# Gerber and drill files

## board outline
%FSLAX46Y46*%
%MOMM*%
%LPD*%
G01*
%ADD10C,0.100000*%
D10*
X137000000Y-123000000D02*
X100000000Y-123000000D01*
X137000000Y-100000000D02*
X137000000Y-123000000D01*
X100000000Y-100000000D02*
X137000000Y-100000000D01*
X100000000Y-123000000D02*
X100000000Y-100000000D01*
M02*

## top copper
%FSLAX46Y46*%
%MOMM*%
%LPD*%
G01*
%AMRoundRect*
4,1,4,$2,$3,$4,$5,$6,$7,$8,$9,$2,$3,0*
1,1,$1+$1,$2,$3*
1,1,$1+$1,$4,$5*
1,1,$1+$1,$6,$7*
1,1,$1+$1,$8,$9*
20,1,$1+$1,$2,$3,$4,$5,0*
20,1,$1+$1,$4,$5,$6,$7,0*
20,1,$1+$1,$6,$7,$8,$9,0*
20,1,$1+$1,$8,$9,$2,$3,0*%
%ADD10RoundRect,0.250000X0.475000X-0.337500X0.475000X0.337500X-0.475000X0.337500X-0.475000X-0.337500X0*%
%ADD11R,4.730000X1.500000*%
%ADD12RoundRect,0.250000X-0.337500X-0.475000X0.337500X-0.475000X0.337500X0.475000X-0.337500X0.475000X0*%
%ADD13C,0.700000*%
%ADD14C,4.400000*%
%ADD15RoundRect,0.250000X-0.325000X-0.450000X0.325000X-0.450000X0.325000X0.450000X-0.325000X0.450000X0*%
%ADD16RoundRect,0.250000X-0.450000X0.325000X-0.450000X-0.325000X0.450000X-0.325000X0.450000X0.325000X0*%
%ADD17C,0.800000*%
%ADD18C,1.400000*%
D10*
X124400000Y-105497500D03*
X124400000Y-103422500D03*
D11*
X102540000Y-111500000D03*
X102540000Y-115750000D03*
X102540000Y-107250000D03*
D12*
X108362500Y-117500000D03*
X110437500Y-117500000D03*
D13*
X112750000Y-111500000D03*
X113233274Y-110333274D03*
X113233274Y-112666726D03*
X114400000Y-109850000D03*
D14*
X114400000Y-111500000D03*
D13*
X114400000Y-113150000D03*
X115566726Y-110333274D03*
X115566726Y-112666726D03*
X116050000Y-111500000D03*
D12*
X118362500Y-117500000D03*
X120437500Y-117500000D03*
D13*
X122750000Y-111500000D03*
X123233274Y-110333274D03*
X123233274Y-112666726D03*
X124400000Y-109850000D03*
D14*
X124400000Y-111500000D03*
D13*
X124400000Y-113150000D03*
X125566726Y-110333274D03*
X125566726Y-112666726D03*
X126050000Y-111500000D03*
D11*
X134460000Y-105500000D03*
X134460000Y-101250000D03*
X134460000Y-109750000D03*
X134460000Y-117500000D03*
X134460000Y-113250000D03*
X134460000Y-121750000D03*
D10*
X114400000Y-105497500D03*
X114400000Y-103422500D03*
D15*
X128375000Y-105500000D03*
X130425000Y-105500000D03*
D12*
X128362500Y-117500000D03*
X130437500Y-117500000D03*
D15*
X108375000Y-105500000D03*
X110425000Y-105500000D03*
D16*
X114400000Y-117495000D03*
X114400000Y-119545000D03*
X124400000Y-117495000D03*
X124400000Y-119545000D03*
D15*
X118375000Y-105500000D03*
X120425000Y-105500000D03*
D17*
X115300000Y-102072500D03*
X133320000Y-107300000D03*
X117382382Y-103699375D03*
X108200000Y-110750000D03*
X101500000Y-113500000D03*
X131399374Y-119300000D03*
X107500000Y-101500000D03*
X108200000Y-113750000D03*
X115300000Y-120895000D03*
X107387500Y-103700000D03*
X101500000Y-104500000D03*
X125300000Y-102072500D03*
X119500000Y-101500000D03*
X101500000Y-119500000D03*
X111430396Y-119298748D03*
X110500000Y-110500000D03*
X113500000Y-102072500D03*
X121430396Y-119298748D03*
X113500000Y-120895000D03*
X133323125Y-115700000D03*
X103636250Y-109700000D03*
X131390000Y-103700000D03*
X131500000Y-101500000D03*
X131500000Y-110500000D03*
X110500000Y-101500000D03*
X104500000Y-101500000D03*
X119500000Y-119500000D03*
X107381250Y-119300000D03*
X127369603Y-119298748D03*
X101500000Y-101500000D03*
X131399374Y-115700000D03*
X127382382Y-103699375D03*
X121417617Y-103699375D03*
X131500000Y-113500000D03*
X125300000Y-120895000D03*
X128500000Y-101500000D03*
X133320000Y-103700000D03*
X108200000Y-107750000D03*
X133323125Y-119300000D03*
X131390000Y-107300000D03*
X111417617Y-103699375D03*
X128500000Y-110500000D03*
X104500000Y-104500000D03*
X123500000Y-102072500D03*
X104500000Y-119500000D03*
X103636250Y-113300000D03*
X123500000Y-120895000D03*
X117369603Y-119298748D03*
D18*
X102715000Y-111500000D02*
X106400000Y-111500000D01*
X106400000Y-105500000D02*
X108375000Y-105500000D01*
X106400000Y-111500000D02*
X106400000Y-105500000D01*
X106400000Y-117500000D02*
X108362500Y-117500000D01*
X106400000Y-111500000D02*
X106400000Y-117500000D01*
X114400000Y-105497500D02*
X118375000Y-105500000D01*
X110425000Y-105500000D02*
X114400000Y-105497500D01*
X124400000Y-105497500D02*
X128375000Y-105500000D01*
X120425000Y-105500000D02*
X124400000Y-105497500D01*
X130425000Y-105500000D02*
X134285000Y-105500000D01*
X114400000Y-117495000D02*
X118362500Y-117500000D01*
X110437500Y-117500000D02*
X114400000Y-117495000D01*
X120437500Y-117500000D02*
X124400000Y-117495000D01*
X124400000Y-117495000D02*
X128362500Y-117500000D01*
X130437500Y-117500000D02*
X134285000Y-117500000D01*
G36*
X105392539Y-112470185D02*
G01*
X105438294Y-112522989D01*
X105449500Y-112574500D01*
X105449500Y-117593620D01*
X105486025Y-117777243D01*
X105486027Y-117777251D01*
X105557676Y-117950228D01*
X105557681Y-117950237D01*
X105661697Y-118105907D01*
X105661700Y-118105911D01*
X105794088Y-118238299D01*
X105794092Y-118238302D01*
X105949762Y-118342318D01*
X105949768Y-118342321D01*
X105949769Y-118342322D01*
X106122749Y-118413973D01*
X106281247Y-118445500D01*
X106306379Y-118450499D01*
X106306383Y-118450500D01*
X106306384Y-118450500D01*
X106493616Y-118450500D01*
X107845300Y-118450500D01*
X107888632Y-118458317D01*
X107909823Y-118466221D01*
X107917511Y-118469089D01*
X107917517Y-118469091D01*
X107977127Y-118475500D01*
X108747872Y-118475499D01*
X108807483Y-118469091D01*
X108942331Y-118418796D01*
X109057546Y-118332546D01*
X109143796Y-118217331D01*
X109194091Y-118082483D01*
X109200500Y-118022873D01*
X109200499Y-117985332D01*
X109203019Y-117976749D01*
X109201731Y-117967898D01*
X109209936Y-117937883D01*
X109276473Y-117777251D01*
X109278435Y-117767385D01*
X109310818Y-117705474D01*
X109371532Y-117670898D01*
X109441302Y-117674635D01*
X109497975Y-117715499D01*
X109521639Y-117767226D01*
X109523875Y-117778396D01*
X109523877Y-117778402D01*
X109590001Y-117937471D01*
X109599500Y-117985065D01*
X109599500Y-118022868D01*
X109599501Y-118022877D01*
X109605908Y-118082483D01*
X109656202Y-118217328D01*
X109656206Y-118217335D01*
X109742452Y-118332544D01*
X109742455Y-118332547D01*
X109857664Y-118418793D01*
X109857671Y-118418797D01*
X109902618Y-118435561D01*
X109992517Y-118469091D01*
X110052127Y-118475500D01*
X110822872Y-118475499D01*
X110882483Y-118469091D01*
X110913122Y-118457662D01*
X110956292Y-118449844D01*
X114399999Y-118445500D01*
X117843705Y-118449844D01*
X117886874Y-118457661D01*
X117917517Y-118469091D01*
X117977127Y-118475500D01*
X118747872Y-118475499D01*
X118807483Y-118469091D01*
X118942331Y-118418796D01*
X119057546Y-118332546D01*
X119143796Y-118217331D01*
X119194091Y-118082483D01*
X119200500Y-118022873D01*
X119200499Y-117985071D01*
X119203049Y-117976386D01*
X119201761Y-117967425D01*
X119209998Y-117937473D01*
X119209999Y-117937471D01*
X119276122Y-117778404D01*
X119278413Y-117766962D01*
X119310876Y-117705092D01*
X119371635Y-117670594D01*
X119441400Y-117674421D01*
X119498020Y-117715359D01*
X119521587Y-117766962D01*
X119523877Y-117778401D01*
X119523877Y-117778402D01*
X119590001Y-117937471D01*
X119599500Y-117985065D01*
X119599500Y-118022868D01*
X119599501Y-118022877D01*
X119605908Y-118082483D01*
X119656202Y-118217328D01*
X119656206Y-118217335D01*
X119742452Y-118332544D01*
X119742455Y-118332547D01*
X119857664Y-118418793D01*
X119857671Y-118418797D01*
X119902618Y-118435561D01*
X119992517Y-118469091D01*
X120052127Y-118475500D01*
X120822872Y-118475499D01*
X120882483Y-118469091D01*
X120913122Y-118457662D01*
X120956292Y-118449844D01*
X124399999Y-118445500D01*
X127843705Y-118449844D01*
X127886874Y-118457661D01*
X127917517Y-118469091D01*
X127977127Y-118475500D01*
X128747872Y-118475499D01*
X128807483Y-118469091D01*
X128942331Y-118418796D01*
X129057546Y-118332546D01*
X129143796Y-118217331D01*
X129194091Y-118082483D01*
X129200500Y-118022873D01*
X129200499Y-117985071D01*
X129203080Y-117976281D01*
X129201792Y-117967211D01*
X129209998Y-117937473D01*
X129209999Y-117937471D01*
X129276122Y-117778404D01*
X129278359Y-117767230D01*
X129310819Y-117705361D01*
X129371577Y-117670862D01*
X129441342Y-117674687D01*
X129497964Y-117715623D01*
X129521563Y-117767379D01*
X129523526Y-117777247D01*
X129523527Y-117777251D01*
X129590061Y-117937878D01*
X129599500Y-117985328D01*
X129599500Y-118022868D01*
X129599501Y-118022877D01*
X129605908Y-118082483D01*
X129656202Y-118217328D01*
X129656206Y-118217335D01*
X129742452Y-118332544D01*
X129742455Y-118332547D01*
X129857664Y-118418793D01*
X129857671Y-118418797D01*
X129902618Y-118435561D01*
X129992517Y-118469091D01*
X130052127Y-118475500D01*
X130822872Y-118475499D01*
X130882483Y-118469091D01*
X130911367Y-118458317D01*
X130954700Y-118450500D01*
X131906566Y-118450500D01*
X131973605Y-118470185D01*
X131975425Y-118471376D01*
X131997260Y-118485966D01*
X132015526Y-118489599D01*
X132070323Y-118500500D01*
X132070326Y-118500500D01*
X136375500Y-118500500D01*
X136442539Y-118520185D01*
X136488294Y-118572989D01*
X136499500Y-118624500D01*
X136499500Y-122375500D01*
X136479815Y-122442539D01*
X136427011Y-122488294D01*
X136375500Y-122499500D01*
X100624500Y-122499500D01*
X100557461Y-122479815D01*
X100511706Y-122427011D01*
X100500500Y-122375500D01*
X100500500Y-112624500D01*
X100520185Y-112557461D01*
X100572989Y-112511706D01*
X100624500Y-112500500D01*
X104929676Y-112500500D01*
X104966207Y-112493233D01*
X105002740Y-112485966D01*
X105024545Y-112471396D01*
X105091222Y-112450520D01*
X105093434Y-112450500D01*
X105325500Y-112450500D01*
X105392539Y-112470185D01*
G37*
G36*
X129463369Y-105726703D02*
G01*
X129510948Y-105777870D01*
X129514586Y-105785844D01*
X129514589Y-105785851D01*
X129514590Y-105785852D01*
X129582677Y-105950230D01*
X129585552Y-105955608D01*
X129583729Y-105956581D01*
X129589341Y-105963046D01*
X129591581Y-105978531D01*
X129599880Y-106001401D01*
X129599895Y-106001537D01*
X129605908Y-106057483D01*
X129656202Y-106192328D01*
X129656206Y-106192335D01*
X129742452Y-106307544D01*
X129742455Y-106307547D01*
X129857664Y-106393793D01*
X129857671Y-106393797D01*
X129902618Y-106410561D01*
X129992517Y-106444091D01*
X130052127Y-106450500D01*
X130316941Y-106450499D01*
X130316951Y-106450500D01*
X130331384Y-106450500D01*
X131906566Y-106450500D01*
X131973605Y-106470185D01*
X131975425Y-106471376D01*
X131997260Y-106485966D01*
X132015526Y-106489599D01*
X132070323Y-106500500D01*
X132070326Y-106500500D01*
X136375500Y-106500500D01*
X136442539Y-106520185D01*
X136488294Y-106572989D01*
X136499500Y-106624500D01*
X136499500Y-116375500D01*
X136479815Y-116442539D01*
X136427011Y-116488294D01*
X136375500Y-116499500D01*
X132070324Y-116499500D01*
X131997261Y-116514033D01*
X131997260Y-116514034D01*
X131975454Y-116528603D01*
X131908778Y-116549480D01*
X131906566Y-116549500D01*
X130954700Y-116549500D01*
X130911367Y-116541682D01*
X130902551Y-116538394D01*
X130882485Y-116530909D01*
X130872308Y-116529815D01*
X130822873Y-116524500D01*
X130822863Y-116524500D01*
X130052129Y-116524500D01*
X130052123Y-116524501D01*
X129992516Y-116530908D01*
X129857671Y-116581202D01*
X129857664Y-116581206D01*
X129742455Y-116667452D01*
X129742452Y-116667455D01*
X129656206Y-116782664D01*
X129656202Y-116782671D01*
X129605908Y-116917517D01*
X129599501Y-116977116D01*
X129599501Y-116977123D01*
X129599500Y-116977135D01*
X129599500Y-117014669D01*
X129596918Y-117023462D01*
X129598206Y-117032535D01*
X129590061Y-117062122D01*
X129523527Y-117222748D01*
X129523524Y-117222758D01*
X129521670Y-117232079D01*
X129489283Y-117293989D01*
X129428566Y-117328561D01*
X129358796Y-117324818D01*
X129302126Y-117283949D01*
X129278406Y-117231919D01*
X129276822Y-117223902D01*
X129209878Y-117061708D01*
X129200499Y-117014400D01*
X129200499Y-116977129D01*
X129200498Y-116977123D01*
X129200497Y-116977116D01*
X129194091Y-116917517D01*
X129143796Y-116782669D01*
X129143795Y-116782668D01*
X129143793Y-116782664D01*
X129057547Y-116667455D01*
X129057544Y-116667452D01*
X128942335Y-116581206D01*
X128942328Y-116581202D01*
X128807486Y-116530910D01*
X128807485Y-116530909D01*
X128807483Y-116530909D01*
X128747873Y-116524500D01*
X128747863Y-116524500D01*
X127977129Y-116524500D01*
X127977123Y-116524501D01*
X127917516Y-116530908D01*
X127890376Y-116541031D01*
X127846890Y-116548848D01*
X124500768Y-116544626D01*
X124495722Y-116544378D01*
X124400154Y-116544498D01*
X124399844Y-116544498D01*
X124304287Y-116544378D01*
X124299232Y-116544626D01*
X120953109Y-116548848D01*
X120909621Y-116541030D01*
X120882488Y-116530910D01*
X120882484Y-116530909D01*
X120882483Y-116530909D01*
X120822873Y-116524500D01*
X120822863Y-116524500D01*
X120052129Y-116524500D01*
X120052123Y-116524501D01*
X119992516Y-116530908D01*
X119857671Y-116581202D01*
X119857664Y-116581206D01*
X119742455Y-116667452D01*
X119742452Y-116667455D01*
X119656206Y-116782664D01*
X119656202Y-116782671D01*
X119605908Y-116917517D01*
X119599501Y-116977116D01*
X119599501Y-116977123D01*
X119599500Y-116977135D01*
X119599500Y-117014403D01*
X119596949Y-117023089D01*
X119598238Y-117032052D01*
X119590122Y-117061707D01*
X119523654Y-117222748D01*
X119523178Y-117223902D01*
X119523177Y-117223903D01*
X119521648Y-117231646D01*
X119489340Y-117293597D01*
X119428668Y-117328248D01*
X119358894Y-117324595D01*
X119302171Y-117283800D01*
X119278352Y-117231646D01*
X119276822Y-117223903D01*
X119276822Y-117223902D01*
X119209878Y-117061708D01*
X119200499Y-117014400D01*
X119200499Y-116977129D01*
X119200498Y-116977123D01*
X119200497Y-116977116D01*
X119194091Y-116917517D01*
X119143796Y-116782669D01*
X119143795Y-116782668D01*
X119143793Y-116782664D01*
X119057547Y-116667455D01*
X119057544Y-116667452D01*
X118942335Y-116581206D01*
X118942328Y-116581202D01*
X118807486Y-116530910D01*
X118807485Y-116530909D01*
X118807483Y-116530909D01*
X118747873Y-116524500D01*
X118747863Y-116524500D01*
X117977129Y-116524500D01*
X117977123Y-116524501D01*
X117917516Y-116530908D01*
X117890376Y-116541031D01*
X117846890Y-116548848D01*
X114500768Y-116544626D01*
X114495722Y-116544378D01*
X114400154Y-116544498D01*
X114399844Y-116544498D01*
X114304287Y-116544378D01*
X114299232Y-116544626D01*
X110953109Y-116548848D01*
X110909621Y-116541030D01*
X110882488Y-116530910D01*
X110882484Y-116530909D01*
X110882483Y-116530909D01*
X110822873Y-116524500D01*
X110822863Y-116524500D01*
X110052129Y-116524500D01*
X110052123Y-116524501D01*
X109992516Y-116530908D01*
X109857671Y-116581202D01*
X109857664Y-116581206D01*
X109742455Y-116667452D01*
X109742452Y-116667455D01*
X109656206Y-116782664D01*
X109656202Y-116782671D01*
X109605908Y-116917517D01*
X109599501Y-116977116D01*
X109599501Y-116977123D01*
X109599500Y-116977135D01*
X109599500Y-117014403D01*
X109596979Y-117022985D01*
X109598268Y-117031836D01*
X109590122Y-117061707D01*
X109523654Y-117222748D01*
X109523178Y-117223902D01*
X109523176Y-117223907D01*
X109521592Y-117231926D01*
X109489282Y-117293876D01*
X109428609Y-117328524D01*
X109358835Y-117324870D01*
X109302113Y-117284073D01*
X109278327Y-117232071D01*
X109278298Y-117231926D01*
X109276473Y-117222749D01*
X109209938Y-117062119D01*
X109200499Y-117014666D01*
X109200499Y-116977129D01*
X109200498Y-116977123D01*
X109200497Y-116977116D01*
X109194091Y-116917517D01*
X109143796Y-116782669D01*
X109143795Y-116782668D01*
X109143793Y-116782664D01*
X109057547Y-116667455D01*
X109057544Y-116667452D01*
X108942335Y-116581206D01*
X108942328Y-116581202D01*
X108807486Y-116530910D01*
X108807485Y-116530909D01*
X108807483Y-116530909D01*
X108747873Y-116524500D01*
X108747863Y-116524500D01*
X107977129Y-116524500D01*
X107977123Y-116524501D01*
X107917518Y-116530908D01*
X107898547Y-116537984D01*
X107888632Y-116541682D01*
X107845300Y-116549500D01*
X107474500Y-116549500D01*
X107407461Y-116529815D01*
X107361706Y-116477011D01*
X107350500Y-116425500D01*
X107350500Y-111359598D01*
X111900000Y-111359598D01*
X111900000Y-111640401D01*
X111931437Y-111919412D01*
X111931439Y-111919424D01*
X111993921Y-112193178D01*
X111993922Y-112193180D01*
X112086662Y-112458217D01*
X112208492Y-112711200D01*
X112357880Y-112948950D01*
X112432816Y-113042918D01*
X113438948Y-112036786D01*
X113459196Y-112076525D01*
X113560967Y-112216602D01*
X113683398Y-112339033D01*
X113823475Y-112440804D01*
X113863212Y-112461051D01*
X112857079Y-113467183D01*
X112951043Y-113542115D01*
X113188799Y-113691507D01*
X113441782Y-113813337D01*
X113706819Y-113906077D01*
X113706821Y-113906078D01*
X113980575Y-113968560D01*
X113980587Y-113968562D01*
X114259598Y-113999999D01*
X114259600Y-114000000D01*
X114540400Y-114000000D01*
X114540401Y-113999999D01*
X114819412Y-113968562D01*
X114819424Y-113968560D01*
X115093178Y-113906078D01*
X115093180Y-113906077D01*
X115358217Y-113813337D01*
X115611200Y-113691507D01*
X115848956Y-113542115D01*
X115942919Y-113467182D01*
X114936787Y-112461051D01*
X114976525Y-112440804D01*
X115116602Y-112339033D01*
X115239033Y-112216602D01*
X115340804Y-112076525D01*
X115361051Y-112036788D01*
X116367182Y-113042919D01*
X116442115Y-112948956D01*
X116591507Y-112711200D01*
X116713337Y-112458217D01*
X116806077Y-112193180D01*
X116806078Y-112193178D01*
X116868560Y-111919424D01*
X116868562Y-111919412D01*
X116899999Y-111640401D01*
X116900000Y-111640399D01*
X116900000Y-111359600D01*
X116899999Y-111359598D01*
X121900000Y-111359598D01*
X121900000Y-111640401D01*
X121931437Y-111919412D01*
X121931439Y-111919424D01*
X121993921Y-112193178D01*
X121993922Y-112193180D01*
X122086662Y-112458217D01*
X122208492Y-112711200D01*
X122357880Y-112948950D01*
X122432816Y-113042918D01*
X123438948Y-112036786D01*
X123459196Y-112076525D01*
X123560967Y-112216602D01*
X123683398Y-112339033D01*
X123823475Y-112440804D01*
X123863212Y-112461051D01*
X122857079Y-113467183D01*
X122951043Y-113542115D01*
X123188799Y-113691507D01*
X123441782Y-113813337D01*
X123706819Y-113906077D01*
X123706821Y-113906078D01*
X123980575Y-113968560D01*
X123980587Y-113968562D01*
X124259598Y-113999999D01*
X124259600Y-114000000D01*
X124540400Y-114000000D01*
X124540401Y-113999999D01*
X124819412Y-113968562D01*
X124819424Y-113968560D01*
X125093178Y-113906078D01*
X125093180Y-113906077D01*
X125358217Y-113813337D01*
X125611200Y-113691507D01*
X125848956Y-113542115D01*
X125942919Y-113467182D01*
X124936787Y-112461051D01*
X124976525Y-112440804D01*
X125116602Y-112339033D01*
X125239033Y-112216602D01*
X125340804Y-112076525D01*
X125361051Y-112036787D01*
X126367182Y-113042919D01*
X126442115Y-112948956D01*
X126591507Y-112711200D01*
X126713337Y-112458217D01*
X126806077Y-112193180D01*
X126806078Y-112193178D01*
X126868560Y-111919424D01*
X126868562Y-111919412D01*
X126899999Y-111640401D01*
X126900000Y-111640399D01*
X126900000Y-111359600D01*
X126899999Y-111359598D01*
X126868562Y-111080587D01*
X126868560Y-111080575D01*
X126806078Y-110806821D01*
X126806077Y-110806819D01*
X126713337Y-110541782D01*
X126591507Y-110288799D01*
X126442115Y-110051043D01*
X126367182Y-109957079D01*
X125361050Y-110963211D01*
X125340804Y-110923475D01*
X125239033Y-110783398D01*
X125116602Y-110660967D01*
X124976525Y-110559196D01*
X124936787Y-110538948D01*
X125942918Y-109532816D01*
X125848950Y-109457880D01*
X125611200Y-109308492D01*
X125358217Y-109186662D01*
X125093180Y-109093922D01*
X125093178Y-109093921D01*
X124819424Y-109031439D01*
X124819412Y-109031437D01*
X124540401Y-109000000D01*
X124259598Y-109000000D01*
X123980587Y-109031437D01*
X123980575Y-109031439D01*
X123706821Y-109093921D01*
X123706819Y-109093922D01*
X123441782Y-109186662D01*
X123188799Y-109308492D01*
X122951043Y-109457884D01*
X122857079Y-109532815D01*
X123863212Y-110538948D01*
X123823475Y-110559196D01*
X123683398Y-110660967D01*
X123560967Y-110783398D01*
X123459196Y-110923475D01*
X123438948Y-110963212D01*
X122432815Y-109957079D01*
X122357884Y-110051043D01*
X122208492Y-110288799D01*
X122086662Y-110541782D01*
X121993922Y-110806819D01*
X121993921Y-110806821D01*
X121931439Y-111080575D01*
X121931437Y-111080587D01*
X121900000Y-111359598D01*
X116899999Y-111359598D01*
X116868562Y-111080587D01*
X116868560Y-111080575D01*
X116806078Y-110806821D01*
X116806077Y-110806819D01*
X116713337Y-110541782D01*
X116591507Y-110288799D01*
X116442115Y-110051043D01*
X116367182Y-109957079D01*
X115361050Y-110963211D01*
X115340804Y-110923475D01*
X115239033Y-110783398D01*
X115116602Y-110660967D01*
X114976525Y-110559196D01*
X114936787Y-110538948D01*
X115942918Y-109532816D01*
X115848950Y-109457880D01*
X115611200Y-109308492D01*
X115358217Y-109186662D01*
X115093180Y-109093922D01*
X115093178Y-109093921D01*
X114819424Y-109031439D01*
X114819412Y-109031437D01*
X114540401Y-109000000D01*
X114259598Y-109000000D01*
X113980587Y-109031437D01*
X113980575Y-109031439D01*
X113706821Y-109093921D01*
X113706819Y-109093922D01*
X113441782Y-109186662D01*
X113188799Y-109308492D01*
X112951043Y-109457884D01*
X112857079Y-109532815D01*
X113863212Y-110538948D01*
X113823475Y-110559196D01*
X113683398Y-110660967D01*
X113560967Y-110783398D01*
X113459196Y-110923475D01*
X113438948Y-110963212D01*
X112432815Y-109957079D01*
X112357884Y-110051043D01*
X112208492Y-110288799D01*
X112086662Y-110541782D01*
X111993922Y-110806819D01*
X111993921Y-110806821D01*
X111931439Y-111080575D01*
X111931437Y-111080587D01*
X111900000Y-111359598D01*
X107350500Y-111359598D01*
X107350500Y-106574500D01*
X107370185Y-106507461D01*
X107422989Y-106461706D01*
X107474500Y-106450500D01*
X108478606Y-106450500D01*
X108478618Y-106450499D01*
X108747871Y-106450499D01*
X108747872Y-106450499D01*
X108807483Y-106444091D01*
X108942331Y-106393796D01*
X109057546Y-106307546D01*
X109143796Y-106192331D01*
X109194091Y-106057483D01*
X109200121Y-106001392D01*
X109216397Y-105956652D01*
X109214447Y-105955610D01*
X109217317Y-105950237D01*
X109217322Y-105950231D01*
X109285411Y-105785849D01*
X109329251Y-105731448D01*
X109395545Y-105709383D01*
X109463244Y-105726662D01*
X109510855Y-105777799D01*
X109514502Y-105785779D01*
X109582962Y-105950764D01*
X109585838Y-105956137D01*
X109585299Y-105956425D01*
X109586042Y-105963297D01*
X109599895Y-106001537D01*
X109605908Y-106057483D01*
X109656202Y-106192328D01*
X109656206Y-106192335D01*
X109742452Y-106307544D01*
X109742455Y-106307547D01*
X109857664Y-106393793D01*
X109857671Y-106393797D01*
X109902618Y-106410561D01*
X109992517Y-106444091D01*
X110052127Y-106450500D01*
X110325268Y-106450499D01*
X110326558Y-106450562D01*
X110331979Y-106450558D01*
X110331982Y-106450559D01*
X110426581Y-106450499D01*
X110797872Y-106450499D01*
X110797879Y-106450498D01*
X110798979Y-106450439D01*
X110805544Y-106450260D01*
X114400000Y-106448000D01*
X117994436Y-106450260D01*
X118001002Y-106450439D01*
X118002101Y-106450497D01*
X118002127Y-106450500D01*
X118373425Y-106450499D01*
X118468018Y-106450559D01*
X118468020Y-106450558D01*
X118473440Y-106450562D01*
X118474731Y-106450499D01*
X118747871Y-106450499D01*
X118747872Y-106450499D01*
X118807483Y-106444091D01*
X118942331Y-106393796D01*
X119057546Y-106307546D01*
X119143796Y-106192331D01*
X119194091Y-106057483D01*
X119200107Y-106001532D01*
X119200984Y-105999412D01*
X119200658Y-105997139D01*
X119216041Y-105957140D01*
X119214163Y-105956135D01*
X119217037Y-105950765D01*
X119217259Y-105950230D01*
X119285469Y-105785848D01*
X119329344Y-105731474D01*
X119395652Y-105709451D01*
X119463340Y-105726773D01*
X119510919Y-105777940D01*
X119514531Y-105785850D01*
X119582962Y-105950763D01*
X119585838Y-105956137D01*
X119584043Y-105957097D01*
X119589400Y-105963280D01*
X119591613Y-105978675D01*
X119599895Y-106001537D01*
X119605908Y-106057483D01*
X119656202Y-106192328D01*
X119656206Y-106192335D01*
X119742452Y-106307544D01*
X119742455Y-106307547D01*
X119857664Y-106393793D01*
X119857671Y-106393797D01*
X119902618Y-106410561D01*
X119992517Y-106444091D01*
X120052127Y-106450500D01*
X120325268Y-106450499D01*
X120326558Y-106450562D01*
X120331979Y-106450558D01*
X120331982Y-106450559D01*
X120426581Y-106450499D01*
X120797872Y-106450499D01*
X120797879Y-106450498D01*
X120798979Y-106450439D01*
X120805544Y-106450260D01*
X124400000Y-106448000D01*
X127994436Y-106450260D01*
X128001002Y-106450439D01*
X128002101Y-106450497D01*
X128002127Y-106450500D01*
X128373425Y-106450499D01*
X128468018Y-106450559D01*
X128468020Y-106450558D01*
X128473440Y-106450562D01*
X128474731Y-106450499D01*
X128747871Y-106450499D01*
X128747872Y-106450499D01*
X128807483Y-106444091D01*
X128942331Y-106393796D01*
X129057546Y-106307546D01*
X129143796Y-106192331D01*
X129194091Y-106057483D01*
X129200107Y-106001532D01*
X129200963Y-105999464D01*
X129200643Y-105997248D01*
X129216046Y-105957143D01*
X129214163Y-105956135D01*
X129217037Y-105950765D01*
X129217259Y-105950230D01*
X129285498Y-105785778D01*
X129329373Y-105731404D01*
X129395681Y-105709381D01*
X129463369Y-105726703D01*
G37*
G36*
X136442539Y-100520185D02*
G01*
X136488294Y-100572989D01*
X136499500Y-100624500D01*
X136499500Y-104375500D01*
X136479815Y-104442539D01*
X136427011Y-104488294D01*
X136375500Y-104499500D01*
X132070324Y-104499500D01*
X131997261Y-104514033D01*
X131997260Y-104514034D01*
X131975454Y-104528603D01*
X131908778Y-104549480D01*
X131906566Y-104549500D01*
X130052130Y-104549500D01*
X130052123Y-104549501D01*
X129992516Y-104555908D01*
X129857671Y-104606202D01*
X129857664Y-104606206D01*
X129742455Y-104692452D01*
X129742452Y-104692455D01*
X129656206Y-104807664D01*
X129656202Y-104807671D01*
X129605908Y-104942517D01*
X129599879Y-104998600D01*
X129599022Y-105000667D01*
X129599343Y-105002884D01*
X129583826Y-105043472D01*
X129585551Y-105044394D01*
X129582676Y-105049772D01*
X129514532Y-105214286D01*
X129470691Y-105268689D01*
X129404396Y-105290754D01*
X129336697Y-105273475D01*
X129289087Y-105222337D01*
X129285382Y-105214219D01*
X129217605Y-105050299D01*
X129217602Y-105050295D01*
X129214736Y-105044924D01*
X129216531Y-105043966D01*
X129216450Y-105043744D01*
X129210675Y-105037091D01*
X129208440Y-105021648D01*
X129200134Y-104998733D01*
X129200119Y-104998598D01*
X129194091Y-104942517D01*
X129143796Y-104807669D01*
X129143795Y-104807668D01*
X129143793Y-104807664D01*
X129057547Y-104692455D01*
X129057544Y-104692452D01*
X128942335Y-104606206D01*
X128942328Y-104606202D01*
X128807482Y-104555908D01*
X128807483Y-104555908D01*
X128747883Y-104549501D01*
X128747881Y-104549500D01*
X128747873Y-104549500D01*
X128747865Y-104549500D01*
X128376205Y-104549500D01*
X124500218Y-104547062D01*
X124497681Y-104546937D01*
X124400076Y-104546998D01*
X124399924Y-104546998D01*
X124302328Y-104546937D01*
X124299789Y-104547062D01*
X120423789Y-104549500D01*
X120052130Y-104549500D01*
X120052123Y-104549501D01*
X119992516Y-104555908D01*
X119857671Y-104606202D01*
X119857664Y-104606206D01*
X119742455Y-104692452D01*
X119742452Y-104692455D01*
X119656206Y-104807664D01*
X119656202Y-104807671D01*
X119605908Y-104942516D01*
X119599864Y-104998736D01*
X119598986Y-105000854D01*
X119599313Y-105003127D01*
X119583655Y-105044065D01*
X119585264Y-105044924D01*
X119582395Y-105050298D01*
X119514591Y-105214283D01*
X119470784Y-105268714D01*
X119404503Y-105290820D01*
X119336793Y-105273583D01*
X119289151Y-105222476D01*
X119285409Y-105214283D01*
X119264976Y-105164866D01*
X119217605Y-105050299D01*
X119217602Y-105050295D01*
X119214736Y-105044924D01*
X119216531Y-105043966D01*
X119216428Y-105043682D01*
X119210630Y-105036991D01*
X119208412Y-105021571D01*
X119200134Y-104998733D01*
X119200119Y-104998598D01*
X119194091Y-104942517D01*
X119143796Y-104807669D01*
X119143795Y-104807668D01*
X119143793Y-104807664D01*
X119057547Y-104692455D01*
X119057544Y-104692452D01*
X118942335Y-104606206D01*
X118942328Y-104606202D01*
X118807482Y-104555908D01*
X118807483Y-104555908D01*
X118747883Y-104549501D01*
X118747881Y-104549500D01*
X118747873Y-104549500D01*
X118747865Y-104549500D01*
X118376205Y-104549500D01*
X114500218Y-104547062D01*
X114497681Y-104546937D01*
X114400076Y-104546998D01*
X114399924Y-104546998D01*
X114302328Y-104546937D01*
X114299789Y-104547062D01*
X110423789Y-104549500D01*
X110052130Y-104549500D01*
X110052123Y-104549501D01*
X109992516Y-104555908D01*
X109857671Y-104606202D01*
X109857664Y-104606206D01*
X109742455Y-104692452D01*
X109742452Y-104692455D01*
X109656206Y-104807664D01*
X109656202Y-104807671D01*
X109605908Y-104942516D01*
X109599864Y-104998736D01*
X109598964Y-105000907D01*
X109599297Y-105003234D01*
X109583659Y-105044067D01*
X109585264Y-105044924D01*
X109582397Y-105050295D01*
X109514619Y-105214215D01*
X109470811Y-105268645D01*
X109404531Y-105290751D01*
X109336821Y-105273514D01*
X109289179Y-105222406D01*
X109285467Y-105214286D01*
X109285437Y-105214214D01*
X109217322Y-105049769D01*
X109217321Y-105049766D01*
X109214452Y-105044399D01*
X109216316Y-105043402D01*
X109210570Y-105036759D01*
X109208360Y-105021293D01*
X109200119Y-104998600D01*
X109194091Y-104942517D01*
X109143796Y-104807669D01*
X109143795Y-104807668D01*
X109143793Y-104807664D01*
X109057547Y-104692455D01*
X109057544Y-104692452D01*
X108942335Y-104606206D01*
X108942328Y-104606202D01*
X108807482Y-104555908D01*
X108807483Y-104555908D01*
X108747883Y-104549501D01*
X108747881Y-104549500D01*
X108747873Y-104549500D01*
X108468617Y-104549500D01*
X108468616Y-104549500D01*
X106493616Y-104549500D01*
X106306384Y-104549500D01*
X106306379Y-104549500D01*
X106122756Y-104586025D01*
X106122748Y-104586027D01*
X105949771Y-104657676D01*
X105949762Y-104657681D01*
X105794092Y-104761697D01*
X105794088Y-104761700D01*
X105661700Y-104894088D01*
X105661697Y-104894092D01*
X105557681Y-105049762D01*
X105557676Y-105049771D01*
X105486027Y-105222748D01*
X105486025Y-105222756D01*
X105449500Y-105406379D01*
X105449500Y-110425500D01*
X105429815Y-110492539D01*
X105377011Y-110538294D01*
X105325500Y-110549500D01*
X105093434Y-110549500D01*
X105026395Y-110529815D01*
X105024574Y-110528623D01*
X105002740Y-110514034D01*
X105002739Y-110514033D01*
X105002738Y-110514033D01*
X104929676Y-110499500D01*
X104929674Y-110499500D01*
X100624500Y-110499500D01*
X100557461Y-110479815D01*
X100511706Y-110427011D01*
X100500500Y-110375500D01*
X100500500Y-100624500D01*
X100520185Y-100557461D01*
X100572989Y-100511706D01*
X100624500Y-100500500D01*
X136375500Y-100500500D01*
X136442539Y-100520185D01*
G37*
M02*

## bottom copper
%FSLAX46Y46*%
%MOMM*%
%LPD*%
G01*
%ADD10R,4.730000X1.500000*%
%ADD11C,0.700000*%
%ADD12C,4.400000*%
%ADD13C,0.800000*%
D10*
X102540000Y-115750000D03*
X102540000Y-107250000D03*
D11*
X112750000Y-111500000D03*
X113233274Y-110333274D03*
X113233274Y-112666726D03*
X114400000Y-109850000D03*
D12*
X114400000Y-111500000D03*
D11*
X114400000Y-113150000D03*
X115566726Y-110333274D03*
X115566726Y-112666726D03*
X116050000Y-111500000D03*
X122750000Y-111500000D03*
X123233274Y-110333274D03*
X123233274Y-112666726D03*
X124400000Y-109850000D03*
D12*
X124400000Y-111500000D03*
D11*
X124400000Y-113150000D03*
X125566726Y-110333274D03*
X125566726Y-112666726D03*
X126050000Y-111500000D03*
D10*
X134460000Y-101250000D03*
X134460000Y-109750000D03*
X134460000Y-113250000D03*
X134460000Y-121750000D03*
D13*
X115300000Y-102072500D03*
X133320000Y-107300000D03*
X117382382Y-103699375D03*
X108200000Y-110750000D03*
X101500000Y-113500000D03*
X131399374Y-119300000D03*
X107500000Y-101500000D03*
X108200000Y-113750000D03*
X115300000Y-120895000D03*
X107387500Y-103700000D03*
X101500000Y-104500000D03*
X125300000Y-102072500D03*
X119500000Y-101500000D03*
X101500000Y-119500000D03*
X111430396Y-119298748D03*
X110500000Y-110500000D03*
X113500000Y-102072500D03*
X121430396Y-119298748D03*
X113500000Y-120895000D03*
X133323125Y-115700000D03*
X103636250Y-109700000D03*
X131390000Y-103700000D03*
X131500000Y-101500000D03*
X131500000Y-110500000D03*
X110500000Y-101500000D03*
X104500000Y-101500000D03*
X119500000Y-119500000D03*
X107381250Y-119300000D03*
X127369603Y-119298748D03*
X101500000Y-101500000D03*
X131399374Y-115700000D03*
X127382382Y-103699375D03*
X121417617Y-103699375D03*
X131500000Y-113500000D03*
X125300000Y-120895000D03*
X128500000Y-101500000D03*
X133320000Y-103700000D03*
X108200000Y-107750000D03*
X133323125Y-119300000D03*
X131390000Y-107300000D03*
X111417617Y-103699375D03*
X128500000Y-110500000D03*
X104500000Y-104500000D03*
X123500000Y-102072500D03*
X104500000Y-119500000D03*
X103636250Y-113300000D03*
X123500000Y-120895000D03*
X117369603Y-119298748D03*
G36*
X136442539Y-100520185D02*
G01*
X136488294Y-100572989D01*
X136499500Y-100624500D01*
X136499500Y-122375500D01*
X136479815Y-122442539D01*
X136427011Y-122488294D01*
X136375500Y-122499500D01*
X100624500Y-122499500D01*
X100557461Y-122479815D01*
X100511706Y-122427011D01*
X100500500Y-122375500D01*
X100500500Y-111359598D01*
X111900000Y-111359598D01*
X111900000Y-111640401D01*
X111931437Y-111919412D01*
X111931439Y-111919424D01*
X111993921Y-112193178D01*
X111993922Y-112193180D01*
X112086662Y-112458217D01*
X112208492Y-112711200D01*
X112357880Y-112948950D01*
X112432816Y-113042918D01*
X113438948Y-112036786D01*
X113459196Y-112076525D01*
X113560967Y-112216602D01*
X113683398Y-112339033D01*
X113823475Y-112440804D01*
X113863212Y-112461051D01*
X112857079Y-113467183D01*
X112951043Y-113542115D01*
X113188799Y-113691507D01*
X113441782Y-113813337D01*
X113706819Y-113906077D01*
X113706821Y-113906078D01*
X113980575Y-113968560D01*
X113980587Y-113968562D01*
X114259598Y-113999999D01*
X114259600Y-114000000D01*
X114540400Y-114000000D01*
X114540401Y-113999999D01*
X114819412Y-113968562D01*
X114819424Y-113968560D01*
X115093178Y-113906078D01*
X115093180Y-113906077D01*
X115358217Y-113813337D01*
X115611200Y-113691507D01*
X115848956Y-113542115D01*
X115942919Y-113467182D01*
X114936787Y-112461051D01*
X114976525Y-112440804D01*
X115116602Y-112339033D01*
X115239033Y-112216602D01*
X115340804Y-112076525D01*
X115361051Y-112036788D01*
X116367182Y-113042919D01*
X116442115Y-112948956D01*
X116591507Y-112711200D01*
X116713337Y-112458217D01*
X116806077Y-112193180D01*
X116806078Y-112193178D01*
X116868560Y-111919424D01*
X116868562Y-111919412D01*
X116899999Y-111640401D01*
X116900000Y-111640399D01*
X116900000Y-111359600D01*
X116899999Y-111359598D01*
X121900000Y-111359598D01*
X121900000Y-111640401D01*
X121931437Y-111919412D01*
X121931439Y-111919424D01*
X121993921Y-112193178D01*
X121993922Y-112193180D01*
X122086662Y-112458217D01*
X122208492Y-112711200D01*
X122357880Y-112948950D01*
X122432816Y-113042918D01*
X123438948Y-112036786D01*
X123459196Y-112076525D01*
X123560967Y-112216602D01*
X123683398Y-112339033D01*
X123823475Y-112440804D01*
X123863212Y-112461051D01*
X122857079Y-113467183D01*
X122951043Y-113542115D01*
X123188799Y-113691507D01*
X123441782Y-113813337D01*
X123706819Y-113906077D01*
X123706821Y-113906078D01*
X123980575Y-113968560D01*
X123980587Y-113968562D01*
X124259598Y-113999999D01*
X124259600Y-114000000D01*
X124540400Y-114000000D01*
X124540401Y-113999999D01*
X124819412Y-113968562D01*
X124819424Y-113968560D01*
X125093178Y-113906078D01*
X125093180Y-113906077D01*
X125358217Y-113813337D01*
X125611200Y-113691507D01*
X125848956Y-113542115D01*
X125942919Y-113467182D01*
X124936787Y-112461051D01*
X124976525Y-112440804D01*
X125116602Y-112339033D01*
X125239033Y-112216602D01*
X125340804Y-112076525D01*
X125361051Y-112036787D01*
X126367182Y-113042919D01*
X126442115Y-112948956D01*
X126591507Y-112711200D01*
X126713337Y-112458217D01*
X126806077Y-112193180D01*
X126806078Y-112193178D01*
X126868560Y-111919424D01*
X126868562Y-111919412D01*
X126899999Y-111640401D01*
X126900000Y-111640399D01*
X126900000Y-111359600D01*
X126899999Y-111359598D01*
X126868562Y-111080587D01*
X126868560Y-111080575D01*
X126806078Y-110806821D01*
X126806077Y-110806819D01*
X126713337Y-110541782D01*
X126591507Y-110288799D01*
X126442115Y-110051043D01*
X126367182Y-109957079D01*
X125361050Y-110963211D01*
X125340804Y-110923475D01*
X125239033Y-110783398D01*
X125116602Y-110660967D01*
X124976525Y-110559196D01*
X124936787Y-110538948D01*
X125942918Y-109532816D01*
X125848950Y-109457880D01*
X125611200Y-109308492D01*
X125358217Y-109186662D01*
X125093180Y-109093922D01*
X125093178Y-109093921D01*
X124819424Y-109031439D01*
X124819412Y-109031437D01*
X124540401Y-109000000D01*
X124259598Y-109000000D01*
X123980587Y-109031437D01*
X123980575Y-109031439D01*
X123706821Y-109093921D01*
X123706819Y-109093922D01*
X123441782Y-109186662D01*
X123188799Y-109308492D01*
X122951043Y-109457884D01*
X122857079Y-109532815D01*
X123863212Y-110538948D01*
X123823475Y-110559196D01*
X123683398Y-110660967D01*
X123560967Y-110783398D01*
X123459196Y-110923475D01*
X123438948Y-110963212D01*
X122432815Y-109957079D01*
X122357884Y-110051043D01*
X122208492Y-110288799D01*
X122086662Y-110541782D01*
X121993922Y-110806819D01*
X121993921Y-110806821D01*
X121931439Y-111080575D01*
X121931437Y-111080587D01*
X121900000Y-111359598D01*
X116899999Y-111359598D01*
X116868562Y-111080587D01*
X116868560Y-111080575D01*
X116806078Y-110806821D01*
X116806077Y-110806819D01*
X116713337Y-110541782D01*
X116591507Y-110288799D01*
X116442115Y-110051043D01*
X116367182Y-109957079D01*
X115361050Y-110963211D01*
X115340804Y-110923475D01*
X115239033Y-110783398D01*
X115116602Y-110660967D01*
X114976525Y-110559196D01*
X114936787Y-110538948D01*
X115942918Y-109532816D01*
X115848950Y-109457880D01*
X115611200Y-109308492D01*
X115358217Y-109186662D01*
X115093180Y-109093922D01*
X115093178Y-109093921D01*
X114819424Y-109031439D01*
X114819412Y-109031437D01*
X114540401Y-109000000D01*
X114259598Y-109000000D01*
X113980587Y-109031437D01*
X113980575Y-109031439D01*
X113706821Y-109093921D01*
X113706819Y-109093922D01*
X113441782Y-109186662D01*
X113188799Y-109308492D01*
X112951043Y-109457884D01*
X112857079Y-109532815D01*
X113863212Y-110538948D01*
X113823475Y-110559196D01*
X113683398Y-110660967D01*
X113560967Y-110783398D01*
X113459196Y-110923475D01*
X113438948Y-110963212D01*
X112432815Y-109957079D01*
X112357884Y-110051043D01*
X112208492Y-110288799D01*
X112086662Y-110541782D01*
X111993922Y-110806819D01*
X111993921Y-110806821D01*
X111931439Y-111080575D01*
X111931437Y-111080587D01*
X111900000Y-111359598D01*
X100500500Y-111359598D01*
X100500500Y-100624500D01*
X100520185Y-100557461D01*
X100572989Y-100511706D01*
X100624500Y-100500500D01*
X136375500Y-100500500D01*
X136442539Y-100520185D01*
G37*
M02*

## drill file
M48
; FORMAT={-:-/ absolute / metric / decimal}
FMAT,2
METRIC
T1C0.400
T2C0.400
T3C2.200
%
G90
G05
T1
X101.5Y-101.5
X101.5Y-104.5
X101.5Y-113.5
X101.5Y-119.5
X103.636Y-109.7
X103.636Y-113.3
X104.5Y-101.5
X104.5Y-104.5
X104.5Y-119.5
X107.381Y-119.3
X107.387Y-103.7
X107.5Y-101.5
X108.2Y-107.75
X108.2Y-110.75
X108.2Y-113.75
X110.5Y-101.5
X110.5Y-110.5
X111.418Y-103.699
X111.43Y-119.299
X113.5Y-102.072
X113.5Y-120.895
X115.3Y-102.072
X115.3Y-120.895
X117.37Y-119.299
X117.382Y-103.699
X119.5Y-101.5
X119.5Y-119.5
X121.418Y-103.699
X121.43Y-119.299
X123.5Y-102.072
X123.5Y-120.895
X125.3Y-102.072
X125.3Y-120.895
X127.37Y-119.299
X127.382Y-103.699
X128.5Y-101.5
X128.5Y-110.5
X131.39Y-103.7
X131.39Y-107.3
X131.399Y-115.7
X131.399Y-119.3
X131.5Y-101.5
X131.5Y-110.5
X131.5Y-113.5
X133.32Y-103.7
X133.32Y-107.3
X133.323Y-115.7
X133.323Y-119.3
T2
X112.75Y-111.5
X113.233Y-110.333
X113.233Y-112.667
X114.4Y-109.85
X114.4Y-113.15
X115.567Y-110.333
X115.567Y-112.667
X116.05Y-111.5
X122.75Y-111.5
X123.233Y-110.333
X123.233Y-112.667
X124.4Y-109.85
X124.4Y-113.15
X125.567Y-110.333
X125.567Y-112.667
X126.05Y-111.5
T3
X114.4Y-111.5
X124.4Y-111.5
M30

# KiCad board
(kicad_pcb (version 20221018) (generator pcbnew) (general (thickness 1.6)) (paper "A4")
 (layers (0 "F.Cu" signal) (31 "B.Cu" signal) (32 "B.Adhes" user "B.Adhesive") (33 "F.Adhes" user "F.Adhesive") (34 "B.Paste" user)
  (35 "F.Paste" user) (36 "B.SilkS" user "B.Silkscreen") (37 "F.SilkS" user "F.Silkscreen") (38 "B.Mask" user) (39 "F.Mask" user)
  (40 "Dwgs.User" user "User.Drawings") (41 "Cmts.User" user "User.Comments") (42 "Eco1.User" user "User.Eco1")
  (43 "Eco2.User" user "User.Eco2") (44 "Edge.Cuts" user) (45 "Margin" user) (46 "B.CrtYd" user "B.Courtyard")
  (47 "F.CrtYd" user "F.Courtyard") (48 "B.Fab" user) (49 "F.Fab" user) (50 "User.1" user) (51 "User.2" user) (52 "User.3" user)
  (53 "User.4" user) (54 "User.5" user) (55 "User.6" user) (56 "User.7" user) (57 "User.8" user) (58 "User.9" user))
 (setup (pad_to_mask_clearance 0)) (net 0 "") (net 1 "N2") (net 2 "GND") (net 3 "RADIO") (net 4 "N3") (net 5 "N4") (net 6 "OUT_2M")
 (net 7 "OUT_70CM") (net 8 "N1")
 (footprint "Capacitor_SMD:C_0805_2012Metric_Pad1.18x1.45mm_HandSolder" (layer "F.Cu") (at 124.4 104.46 90)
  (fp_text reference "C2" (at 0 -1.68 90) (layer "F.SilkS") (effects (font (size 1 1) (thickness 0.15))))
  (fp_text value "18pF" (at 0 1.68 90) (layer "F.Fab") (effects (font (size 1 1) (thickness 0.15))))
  (pad "1" smd roundrect (at -1.0375 0 90) (size 1.175 1.45) (layers "F.Cu" "F.Paste" "F.Mask") (roundrect_rratio 0.212766) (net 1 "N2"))
  (pad "2" smd roundrect (at 1.0375 0 90) (size 1.175 1.45) (layers "F.Cu" "F.Paste" "F.Mask") (roundrect_rratio 0.212766) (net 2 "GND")))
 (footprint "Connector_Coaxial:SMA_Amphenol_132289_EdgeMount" (layer "F.Cu") (at 102.54 111.5 180)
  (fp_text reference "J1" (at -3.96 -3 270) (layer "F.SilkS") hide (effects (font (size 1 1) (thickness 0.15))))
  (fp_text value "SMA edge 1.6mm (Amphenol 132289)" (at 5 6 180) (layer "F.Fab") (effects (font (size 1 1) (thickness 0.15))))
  (pad "1" smd rect (at 0 0 270) (size 1.5 4.73) (layers "F.Cu" "F.Paste" "F.Mask") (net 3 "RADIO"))
  (pad "2" smd rect (at 0 -4.25 270) (size 1.5 4.73) (layers "F.Cu" "F.Paste" "F.Mask") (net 2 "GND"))
  (pad "2" smd rect (at 0 -4.25 270) (size 1.5 4.73) (layers "B.Cu" "B.Paste" "B.Mask") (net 2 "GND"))
  (pad "2" smd rect (at 0 4.25 270) (size 1.5 4.73) (layers "F.Cu" "F.Paste" "F.Mask") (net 2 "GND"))
  (pad "2" smd rect (at 0 4.25 270) (size 1.5 4.73) (layers "B.Cu" "B.Paste" "B.Mask") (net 2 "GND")))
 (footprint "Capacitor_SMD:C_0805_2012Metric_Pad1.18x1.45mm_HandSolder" (layer "F.Cu") (at 109.4 117.5)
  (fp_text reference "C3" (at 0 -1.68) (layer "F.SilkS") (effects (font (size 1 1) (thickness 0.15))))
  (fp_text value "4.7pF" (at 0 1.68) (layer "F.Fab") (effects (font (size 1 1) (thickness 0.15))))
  (pad "1" smd roundrect (at -1.0375 0) (size 1.175 1.45) (layers "F.Cu" "F.Paste" "F.Mask") (roundrect_rratio 0.212766) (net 3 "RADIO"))
  (pad "2" smd roundrect (at 1.0375 0) (size 1.175 1.45) (layers "F.Cu" "F.Paste" "F.Mask") (roundrect_rratio 0.212766) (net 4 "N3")))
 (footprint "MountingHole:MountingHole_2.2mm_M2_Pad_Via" (layer "F.Cu") (at 114.4 111.5)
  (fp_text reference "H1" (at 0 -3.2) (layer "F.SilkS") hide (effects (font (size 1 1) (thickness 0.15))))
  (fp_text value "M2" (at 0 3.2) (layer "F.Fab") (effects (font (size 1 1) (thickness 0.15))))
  (pad "1" thru_hole circle (at -1.65 0) (size 0.7 0.7) (drill 0.4) (layers "*.Cu" "*.Mask") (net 2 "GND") (zone_connect 2))
  (pad "1" thru_hole circle (at -1.166726 -1.166726) (size 0.7 0.7) (drill 0.4) (layers "*.Cu" "*.Mask") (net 2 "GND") (zone_connect 2))
  (pad "1" thru_hole circle (at -1.166726 1.166726) (size 0.7 0.7) (drill 0.4) (layers "*.Cu" "*.Mask") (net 2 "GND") (zone_connect 2))
  (pad "1" thru_hole circle (at 0 -1.65) (size 0.7 0.7) (drill 0.4) (layers "*.Cu" "*.Mask") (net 2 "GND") (zone_connect 2))
  (pad "1" thru_hole circle (at 0 0) (size 4.4 4.4) (drill 2.2) (layers "*.Cu" "*.Mask") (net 2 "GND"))
  (pad "1" thru_hole circle (at 0 1.65) (size 0.7 0.7) (drill 0.4) (layers "*.Cu" "*.Mask") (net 2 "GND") (zone_connect 2))
  (pad "1" thru_hole circle (at 1.166726 -1.166726) (size 0.7 0.7) (drill 0.4) (layers "*.Cu" "*.Mask") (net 2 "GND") (zone_connect 2))
  (pad "1" thru_hole circle (at 1.166726 1.166726) (size 0.7 0.7) (drill 0.4) (layers "*.Cu" "*.Mask") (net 2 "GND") (zone_connect 2))
  (pad "1" thru_hole circle (at 1.65 0) (size 0.7 0.7) (drill 0.4) (layers "*.Cu" "*.Mask") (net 2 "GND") (zone_connect 2)))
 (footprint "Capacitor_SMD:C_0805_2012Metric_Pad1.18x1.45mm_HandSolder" (layer "F.Cu") (at 119.4 117.5)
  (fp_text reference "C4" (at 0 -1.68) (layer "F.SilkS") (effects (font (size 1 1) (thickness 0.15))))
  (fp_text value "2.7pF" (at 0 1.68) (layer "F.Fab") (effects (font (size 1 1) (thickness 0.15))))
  (pad "1" smd roundrect (at -1.0375 0) (size 1.175 1.45) (layers "F.Cu" "F.Paste" "F.Mask") (roundrect_rratio 0.212766) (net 4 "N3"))
  (pad "2" smd roundrect (at 1.0375 0) (size 1.175 1.45) (layers "F.Cu" "F.Paste" "F.Mask") (roundrect_rratio 0.212766) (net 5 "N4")))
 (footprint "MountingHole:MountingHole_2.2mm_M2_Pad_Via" (layer "F.Cu") (at 124.4 111.5)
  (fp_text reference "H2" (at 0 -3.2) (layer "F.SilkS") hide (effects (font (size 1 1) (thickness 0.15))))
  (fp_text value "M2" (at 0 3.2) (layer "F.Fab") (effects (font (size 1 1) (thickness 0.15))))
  (pad "1" thru_hole circle (at -1.65 0) (size 0.7 0.7) (drill 0.4) (layers "*.Cu" "*.Mask") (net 2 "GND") (zone_connect 2))
  (pad "1" thru_hole circle (at -1.166726 -1.166726) (size 0.7 0.7) (drill 0.4) (layers "*.Cu" "*.Mask") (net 2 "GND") (zone_connect 2))
  (pad "1" thru_hole circle (at -1.166726 1.166726) (size 0.7 0.7) (drill 0.4) (layers "*.Cu" "*.Mask") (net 2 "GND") (zone_connect 2))
  (pad "1" thru_hole circle (at 0 -1.65) (size 0.7 0.7) (drill 0.4) (layers "*.Cu" "*.Mask") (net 2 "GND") (zone_connect 2))
  (pad "1" thru_hole circle (at 0 0) (size 4.4 4.4) (drill 2.2) (layers "*.Cu" "*.Mask") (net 2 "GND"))
  (pad "1" thru_hole circle (at 0 1.65) (size 0.7 0.7) (drill 0.4) (layers "*.Cu" "*.Mask") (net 2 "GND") (zone_connect 2))
  (pad "1" thru_hole circle (at 1.166726 -1.166726) (size 0.7 0.7) (drill 0.4) (layers "*.Cu" "*.Mask") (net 2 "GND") (zone_connect 2))
  (pad "1" thru_hole circle (at 1.166726 1.166726) (size 0.7 0.7) (drill 0.4) (layers "*.Cu" "*.Mask") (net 2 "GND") (zone_connect 2))
  (pad "1" thru_hole circle (at 1.65 0) (size 0.7 0.7) (drill 0.4) (layers "*.Cu" "*.Mask") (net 2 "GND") (zone_connect 2)))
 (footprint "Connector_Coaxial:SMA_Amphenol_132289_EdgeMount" (layer "F.Cu") (at 134.46 105.5)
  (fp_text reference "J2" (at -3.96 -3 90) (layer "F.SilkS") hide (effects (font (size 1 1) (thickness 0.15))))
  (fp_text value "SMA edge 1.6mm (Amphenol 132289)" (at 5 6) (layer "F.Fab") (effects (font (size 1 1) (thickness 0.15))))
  (pad "1" smd rect (at 0 0 90) (size 1.5 4.73) (layers "F.Cu" "F.Paste" "F.Mask") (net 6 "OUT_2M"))
  (pad "2" smd rect (at 0 -4.25 90) (size 1.5 4.73) (layers "F.Cu" "F.Paste" "F.Mask") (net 2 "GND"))
  (pad "2" smd rect (at 0 -4.25 90) (size 1.5 4.73) (layers "B.Cu" "B.Paste" "B.Mask") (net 2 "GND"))
  (pad "2" smd rect (at 0 4.25 90) (size 1.5 4.73) (layers "F.Cu" "F.Paste" "F.Mask") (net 2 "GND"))
  (pad "2" smd rect (at 0 4.25 90) (size 1.5 4.73) (layers "B.Cu" "B.Paste" "B.Mask") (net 2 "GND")))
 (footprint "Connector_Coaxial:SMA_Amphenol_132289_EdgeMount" (layer "F.Cu") (at 134.46 117.5)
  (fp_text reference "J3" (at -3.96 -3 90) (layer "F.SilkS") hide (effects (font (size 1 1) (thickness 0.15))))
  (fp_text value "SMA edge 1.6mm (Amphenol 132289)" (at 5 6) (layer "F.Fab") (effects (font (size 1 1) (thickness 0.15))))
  (pad "1" smd rect (at 0 0 90) (size 1.5 4.73) (layers "F.Cu" "F.Paste" "F.Mask") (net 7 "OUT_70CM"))
  (pad "2" smd rect (at 0 -4.25 90) (size 1.5 4.73) (layers "F.Cu" "F.Paste" "F.Mask") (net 2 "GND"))
  (pad "2" smd rect (at 0 -4.25 90) (size 1.5 4.73) (layers "B.Cu" "B.Paste" "B.Mask") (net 2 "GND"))
  (pad "2" smd rect (at 0 4.25 90) (size 1.5 4.73) (layers "F.Cu" "F.Paste" "F.Mask") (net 2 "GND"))
  (pad "2" smd rect (at 0 4.25 90) (size 1.5 4.73) (layers "B.Cu" "B.Paste" "B.Mask") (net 2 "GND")))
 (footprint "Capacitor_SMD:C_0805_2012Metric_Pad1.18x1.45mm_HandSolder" (layer "F.Cu") (at 114.4 104.46 90)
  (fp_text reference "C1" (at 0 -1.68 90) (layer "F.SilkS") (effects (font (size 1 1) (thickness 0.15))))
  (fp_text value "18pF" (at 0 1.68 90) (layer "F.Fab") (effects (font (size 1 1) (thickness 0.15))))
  (pad "1" smd roundrect (at -1.0375 0 90) (size 1.175 1.45) (layers "F.Cu" "F.Paste" "F.Mask") (roundrect_rratio 0.212766) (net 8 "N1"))
  (pad "2" smd roundrect (at 1.0375 0 90) (size 1.175 1.45) (layers "F.Cu" "F.Paste" "F.Mask") (roundrect_rratio 0.212766) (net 2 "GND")))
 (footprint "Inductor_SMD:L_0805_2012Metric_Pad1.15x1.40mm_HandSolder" (layer "F.Cu") (at 129.4 105.5)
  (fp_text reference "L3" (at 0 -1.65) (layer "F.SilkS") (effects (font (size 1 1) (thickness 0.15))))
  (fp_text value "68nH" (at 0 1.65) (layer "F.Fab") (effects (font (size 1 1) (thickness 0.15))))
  (pad "1" smd roundrect (at -1.025 0) (size 1.15 1.4) (layers "F.Cu" "F.Paste" "F.Mask") (roundrect_rratio 0.217391) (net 1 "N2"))
  (pad "2" smd roundrect (at 1.025 0) (size 1.15 1.4) (layers "F.Cu" "F.Paste" "F.Mask") (roundrect_rratio 0.217391) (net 6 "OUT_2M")))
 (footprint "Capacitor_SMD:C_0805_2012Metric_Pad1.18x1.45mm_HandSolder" (layer "F.Cu") (at 129.4 117.5)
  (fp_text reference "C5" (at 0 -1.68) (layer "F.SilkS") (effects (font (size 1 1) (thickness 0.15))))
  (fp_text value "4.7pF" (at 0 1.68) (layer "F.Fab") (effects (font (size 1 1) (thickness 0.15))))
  (pad "1" smd roundrect (at -1.0375 0) (size 1.175 1.45) (layers "F.Cu" "F.Paste" "F.Mask") (roundrect_rratio 0.212766) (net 5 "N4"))
  (pad "2" smd roundrect (at 1.0375 0) (size 1.175 1.45) (layers "F.Cu" "F.Paste" "F.Mask") (roundrect_rratio 0.212766) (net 7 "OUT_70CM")))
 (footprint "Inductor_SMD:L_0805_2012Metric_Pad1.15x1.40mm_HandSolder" (layer "F.Cu") (at 109.4 105.5)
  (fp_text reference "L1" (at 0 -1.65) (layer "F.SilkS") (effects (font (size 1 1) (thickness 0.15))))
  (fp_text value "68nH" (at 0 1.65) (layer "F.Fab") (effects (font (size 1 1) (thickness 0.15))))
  (pad "1" smd roundrect (at -1.025 0) (size 1.15 1.4) (layers "F.Cu" "F.Paste" "F.Mask") (roundrect_rratio 0.217391) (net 3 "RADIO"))
  (pad "2" smd roundrect (at 1.025 0) (size 1.15 1.4) (layers "F.Cu" "F.Paste" "F.Mask") (roundrect_rratio 0.217391) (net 8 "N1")))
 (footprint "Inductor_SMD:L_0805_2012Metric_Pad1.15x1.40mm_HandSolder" (layer "F.Cu") (at 114.4 118.52 -90)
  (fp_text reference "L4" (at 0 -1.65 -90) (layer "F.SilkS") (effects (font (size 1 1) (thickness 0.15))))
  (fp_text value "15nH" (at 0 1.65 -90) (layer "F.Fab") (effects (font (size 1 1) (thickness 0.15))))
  (pad "1" smd roundrect (at -1.025 0 270) (size 1.15 1.4) (layers "F.Cu" "F.Paste" "F.Mask") (roundrect_rratio 0.217391) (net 4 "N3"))
  (pad "2" smd roundrect (at 1.025 0 270) (size 1.15 1.4) (layers "F.Cu" "F.Paste" "F.Mask") (roundrect_rratio 0.217391) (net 2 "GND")))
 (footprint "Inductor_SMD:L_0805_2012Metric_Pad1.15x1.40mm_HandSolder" (layer "F.Cu") (at 124.4 118.52 -90)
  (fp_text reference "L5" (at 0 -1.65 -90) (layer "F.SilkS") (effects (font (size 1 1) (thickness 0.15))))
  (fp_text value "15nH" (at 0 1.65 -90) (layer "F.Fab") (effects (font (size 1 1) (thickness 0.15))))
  (pad "1" smd roundrect (at -1.025 0 270) (size 1.15 1.4) (layers "F.Cu" "F.Paste" "F.Mask") (roundrect_rratio 0.217391) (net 5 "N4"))
  (pad "2" smd roundrect (at 1.025 0 270) (size 1.15 1.4) (layers "F.Cu" "F.Paste" "F.Mask") (roundrect_rratio 0.217391) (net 2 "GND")))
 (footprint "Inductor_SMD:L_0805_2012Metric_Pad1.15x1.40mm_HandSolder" (layer "F.Cu") (at 119.4 105.5)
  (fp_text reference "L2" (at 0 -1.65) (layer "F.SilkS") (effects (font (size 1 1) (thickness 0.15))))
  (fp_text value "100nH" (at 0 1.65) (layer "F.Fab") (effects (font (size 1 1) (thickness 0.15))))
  (pad "1" smd roundrect (at -1.025 0) (size 1.15 1.4) (layers "F.Cu" "F.Paste" "F.Mask") (roundrect_rratio 0.217391) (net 8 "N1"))
  (pad "2" smd roundrect (at 1.025 0) (size 1.15 1.4) (layers "F.Cu" "F.Paste" "F.Mask") (roundrect_rratio 0.217391) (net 1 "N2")))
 (gr_line (start 137 123) (end 100 123) (stroke (width 0.1) (type default)) (layer "Edge.Cuts"))
 (gr_line (start 137 100) (end 137 123) (stroke (width 0.1) (type default)) (layer "Edge.Cuts"))
 (gr_line (start 100 100) (end 137 100) (stroke (width 0.1) (type default)) (layer "Edge.Cuts"))
 (gr_line (start 100 123) (end 100 100) (stroke (width 0.1) (type default)) (layer "Edge.Cuts"))
 (via (at 115.3 102.0725) (size 0.8) (drill 0.4) (layers "F.Cu" "B.Cu") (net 2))
 (via (at 133.32 107.3) (size 0.8) (drill 0.4) (layers "F.Cu" "B.Cu") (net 2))
 (via (at 117.382382 103.699375) (size 0.8) (drill 0.4) (layers "F.Cu" "B.Cu") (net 2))
 (via (at 108.2 110.75) (size 0.8) (drill 0.4) (layers "F.Cu" "B.Cu") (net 2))
 (via (at 101.5 113.5) (size 0.8) (drill 0.4) (layers "F.Cu" "B.Cu") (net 2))
 (via (at 131.399374 119.3) (size 0.8) (drill 0.4) (layers "F.Cu" "B.Cu") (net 2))
 (via (at 107.5 101.5) (size 0.8) (drill 0.4) (layers "F.Cu" "B.Cu") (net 2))
 (via (at 108.2 113.75) (size 0.8) (drill 0.4) (layers "F.Cu" "B.Cu") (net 2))
 (via (at 115.3 120.895) (size 0.8) (drill 0.4) (layers "F.Cu" "B.Cu") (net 2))
 (via (at 107.3875 103.7) (size 0.8) (drill 0.4) (layers "F.Cu" "B.Cu") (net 2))
 (via (at 101.5 104.5) (size 0.8) (drill 0.4) (layers "F.Cu" "B.Cu") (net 2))
 (via (at 125.3 102.0725) (size 0.8) (drill 0.4) (layers "F.Cu" "B.Cu") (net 2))
 (via (at 119.5 101.5) (size 0.8) (drill 0.4) (layers "F.Cu" "B.Cu") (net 2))
 (via (at 101.5 119.5) (size 0.8) (drill 0.4) (layers "F.Cu" "B.Cu") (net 2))
 (via (at 111.430396 119.298748) (size 0.8) (drill 0.4) (layers "F.Cu" "B.Cu") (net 2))
 (via (at 110.5 110.5) (size 0.8) (drill 0.4) (layers "F.Cu" "B.Cu") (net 2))
 (via (at 113.5 102.0725) (size 0.8) (drill 0.4) (layers "F.Cu" "B.Cu") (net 2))
 (via (at 121.430396 119.298748) (size 0.8) (drill 0.4) (layers "F.Cu" "B.Cu") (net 2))
 (via (at 113.5 120.895) (size 0.8) (drill 0.4) (layers "F.Cu" "B.Cu") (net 2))
 (via (at 133.323125 115.7) (size 0.8) (drill 0.4) (layers "F.Cu" "B.Cu") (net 2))
 (via (at 103.63625 109.7) (size 0.8) (drill 0.4) (layers "F.Cu" "B.Cu") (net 2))
 (via (at 131.39 103.7) (size 0.8) (drill 0.4) (layers "F.Cu" "B.Cu") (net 2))
 (via (at 131.5 101.5) (size 0.8) (drill 0.4) (layers "F.Cu" "B.Cu") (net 2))
 (via (at 131.5 110.5) (size 0.8) (drill 0.4) (layers "F.Cu" "B.Cu") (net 2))
 (via (at 110.5 101.5) (size 0.8) (drill 0.4) (layers "F.Cu" "B.Cu") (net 2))
 (via (at 104.5 101.5) (size 0.8) (drill 0.4) (layers "F.Cu" "B.Cu") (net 2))
 (via (at 119.5 119.5) (size 0.8) (drill 0.4) (layers "F.Cu" "B.Cu") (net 2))
 (via (at 107.38125 119.3) (size 0.8) (drill 0.4) (layers "F.Cu" "B.Cu") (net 2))
 (via (at 127.369603 119.298748) (size 0.8) (drill 0.4) (layers "F.Cu" "B.Cu") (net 2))
 (via (at 101.5 101.5) (size 0.8) (drill 0.4) (layers "F.Cu" "B.Cu") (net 2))
 (via (at 131.399374 115.7) (size 0.8) (drill 0.4) (layers "F.Cu" "B.Cu") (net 2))
 (via (at 127.382382 103.699375) (size 0.8) (drill 0.4) (layers "F.Cu" "B.Cu") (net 2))
 (via (at 121.417617 103.699375) (size 0.8) (drill 0.4) (layers "F.Cu" "B.Cu") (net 2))
 (via (at 131.5 113.5) (size 0.8) (drill 0.4) (layers "F.Cu" "B.Cu") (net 2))
 (via (at 125.3 120.895) (size 0.8) (drill 0.4) (layers "F.Cu" "B.Cu") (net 2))
 (via (at 128.5 101.5) (size 0.8) (drill 0.4) (layers "F.Cu" "B.Cu") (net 2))
 (via (at 133.32 103.7) (size 0.8) (drill 0.4) (layers "F.Cu" "B.Cu") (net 2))
 (via (at 108.2 107.75) (size 0.8) (drill 0.4) (layers "F.Cu" "B.Cu") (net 2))
 (via (at 133.323125 119.3) (size 0.8) (drill 0.4) (layers "F.Cu" "B.Cu") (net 2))
 (via (at 131.39 107.3) (size 0.8) (drill 0.4) (layers "F.Cu" "B.Cu") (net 2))
 (via (at 111.417617 103.699375) (size 0.8) (drill 0.4) (layers "F.Cu" "B.Cu") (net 2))
 (via (at 128.5 110.5) (size 0.8) (drill 0.4) (layers "F.Cu" "B.Cu") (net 2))
 (via (at 104.5 104.5) (size 0.8) (drill 0.4) (layers "F.Cu" "B.Cu") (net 2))
 (via (at 123.5 102.0725) (size 0.8) (drill 0.4) (layers "F.Cu" "B.Cu") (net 2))
 (via (at 104.5 119.5) (size 0.8) (drill 0.4) (layers "F.Cu" "B.Cu") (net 2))
 (via (at 103.63625 113.3) (size 0.8) (drill 0.4) (layers "F.Cu" "B.Cu") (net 2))
 (via (at 123.5 120.895) (size 0.8) (drill 0.4) (layers "F.Cu" "B.Cu") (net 2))
 (via (at 117.369603 119.298748) (size 0.8) (drill 0.4) (layers "F.Cu" "B.Cu") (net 2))
 (segment (start 102.715 111.5) (end 106.4 111.5) (width 1.4) (layer "F.Cu") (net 3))
 (segment (start 106.4 105.5) (end 108.375 105.5) (width 1.4) (layer "F.Cu") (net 3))
 (segment (start 106.4 111.5) (end 106.4 105.5) (width 1.4) (layer "F.Cu") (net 3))
 (segment (start 106.4 117.5) (end 108.3625 117.5) (width 1.4) (layer "F.Cu") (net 3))
 (segment (start 106.4 111.5) (end 106.4 117.5) (width 1.4) (layer "F.Cu") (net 3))
 (segment (start 114.4 105.4975) (end 118.375 105.5) (width 1.4) (layer "F.Cu") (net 8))
 (segment (start 110.425 105.5) (end 114.4 105.4975) (width 1.4) (layer "F.Cu") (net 8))
 (segment (start 124.4 105.4975) (end 128.375 105.5) (width 1.4) (layer "F.Cu") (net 1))
 (segment (start 120.425 105.5) (end 124.4 105.4975) (width 1.4) (layer "F.Cu") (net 1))
 (segment (start 130.425 105.5) (end 134.285 105.5) (width 1.4) (layer "F.Cu") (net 6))
 (segment (start 114.4 117.495) (end 118.3625 117.5) (width 1.4) (layer "F.Cu") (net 4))
 (segment (start 110.4375 117.5) (end 114.4 117.495) (width 1.4) (layer "F.Cu") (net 4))
 (segment (start 120.4375 117.5) (end 124.4 117.495) (width 1.4) (layer "F.Cu") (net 5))
 (segment (start 124.4 117.495) (end 128.3625 117.5) (width 1.4) (layer "F.Cu") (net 5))
 (segment (start 130.4375 117.5) (end 134.285 117.5) (width 1.4) (layer "F.Cu") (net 7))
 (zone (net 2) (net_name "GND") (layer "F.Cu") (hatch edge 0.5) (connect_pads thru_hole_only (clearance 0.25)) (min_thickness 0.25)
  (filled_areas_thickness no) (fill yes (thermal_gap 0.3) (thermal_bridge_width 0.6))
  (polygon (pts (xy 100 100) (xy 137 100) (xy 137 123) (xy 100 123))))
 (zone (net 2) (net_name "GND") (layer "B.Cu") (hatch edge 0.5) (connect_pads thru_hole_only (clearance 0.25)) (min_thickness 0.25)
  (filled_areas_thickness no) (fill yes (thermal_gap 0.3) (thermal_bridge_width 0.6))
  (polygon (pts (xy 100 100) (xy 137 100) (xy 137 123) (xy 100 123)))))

